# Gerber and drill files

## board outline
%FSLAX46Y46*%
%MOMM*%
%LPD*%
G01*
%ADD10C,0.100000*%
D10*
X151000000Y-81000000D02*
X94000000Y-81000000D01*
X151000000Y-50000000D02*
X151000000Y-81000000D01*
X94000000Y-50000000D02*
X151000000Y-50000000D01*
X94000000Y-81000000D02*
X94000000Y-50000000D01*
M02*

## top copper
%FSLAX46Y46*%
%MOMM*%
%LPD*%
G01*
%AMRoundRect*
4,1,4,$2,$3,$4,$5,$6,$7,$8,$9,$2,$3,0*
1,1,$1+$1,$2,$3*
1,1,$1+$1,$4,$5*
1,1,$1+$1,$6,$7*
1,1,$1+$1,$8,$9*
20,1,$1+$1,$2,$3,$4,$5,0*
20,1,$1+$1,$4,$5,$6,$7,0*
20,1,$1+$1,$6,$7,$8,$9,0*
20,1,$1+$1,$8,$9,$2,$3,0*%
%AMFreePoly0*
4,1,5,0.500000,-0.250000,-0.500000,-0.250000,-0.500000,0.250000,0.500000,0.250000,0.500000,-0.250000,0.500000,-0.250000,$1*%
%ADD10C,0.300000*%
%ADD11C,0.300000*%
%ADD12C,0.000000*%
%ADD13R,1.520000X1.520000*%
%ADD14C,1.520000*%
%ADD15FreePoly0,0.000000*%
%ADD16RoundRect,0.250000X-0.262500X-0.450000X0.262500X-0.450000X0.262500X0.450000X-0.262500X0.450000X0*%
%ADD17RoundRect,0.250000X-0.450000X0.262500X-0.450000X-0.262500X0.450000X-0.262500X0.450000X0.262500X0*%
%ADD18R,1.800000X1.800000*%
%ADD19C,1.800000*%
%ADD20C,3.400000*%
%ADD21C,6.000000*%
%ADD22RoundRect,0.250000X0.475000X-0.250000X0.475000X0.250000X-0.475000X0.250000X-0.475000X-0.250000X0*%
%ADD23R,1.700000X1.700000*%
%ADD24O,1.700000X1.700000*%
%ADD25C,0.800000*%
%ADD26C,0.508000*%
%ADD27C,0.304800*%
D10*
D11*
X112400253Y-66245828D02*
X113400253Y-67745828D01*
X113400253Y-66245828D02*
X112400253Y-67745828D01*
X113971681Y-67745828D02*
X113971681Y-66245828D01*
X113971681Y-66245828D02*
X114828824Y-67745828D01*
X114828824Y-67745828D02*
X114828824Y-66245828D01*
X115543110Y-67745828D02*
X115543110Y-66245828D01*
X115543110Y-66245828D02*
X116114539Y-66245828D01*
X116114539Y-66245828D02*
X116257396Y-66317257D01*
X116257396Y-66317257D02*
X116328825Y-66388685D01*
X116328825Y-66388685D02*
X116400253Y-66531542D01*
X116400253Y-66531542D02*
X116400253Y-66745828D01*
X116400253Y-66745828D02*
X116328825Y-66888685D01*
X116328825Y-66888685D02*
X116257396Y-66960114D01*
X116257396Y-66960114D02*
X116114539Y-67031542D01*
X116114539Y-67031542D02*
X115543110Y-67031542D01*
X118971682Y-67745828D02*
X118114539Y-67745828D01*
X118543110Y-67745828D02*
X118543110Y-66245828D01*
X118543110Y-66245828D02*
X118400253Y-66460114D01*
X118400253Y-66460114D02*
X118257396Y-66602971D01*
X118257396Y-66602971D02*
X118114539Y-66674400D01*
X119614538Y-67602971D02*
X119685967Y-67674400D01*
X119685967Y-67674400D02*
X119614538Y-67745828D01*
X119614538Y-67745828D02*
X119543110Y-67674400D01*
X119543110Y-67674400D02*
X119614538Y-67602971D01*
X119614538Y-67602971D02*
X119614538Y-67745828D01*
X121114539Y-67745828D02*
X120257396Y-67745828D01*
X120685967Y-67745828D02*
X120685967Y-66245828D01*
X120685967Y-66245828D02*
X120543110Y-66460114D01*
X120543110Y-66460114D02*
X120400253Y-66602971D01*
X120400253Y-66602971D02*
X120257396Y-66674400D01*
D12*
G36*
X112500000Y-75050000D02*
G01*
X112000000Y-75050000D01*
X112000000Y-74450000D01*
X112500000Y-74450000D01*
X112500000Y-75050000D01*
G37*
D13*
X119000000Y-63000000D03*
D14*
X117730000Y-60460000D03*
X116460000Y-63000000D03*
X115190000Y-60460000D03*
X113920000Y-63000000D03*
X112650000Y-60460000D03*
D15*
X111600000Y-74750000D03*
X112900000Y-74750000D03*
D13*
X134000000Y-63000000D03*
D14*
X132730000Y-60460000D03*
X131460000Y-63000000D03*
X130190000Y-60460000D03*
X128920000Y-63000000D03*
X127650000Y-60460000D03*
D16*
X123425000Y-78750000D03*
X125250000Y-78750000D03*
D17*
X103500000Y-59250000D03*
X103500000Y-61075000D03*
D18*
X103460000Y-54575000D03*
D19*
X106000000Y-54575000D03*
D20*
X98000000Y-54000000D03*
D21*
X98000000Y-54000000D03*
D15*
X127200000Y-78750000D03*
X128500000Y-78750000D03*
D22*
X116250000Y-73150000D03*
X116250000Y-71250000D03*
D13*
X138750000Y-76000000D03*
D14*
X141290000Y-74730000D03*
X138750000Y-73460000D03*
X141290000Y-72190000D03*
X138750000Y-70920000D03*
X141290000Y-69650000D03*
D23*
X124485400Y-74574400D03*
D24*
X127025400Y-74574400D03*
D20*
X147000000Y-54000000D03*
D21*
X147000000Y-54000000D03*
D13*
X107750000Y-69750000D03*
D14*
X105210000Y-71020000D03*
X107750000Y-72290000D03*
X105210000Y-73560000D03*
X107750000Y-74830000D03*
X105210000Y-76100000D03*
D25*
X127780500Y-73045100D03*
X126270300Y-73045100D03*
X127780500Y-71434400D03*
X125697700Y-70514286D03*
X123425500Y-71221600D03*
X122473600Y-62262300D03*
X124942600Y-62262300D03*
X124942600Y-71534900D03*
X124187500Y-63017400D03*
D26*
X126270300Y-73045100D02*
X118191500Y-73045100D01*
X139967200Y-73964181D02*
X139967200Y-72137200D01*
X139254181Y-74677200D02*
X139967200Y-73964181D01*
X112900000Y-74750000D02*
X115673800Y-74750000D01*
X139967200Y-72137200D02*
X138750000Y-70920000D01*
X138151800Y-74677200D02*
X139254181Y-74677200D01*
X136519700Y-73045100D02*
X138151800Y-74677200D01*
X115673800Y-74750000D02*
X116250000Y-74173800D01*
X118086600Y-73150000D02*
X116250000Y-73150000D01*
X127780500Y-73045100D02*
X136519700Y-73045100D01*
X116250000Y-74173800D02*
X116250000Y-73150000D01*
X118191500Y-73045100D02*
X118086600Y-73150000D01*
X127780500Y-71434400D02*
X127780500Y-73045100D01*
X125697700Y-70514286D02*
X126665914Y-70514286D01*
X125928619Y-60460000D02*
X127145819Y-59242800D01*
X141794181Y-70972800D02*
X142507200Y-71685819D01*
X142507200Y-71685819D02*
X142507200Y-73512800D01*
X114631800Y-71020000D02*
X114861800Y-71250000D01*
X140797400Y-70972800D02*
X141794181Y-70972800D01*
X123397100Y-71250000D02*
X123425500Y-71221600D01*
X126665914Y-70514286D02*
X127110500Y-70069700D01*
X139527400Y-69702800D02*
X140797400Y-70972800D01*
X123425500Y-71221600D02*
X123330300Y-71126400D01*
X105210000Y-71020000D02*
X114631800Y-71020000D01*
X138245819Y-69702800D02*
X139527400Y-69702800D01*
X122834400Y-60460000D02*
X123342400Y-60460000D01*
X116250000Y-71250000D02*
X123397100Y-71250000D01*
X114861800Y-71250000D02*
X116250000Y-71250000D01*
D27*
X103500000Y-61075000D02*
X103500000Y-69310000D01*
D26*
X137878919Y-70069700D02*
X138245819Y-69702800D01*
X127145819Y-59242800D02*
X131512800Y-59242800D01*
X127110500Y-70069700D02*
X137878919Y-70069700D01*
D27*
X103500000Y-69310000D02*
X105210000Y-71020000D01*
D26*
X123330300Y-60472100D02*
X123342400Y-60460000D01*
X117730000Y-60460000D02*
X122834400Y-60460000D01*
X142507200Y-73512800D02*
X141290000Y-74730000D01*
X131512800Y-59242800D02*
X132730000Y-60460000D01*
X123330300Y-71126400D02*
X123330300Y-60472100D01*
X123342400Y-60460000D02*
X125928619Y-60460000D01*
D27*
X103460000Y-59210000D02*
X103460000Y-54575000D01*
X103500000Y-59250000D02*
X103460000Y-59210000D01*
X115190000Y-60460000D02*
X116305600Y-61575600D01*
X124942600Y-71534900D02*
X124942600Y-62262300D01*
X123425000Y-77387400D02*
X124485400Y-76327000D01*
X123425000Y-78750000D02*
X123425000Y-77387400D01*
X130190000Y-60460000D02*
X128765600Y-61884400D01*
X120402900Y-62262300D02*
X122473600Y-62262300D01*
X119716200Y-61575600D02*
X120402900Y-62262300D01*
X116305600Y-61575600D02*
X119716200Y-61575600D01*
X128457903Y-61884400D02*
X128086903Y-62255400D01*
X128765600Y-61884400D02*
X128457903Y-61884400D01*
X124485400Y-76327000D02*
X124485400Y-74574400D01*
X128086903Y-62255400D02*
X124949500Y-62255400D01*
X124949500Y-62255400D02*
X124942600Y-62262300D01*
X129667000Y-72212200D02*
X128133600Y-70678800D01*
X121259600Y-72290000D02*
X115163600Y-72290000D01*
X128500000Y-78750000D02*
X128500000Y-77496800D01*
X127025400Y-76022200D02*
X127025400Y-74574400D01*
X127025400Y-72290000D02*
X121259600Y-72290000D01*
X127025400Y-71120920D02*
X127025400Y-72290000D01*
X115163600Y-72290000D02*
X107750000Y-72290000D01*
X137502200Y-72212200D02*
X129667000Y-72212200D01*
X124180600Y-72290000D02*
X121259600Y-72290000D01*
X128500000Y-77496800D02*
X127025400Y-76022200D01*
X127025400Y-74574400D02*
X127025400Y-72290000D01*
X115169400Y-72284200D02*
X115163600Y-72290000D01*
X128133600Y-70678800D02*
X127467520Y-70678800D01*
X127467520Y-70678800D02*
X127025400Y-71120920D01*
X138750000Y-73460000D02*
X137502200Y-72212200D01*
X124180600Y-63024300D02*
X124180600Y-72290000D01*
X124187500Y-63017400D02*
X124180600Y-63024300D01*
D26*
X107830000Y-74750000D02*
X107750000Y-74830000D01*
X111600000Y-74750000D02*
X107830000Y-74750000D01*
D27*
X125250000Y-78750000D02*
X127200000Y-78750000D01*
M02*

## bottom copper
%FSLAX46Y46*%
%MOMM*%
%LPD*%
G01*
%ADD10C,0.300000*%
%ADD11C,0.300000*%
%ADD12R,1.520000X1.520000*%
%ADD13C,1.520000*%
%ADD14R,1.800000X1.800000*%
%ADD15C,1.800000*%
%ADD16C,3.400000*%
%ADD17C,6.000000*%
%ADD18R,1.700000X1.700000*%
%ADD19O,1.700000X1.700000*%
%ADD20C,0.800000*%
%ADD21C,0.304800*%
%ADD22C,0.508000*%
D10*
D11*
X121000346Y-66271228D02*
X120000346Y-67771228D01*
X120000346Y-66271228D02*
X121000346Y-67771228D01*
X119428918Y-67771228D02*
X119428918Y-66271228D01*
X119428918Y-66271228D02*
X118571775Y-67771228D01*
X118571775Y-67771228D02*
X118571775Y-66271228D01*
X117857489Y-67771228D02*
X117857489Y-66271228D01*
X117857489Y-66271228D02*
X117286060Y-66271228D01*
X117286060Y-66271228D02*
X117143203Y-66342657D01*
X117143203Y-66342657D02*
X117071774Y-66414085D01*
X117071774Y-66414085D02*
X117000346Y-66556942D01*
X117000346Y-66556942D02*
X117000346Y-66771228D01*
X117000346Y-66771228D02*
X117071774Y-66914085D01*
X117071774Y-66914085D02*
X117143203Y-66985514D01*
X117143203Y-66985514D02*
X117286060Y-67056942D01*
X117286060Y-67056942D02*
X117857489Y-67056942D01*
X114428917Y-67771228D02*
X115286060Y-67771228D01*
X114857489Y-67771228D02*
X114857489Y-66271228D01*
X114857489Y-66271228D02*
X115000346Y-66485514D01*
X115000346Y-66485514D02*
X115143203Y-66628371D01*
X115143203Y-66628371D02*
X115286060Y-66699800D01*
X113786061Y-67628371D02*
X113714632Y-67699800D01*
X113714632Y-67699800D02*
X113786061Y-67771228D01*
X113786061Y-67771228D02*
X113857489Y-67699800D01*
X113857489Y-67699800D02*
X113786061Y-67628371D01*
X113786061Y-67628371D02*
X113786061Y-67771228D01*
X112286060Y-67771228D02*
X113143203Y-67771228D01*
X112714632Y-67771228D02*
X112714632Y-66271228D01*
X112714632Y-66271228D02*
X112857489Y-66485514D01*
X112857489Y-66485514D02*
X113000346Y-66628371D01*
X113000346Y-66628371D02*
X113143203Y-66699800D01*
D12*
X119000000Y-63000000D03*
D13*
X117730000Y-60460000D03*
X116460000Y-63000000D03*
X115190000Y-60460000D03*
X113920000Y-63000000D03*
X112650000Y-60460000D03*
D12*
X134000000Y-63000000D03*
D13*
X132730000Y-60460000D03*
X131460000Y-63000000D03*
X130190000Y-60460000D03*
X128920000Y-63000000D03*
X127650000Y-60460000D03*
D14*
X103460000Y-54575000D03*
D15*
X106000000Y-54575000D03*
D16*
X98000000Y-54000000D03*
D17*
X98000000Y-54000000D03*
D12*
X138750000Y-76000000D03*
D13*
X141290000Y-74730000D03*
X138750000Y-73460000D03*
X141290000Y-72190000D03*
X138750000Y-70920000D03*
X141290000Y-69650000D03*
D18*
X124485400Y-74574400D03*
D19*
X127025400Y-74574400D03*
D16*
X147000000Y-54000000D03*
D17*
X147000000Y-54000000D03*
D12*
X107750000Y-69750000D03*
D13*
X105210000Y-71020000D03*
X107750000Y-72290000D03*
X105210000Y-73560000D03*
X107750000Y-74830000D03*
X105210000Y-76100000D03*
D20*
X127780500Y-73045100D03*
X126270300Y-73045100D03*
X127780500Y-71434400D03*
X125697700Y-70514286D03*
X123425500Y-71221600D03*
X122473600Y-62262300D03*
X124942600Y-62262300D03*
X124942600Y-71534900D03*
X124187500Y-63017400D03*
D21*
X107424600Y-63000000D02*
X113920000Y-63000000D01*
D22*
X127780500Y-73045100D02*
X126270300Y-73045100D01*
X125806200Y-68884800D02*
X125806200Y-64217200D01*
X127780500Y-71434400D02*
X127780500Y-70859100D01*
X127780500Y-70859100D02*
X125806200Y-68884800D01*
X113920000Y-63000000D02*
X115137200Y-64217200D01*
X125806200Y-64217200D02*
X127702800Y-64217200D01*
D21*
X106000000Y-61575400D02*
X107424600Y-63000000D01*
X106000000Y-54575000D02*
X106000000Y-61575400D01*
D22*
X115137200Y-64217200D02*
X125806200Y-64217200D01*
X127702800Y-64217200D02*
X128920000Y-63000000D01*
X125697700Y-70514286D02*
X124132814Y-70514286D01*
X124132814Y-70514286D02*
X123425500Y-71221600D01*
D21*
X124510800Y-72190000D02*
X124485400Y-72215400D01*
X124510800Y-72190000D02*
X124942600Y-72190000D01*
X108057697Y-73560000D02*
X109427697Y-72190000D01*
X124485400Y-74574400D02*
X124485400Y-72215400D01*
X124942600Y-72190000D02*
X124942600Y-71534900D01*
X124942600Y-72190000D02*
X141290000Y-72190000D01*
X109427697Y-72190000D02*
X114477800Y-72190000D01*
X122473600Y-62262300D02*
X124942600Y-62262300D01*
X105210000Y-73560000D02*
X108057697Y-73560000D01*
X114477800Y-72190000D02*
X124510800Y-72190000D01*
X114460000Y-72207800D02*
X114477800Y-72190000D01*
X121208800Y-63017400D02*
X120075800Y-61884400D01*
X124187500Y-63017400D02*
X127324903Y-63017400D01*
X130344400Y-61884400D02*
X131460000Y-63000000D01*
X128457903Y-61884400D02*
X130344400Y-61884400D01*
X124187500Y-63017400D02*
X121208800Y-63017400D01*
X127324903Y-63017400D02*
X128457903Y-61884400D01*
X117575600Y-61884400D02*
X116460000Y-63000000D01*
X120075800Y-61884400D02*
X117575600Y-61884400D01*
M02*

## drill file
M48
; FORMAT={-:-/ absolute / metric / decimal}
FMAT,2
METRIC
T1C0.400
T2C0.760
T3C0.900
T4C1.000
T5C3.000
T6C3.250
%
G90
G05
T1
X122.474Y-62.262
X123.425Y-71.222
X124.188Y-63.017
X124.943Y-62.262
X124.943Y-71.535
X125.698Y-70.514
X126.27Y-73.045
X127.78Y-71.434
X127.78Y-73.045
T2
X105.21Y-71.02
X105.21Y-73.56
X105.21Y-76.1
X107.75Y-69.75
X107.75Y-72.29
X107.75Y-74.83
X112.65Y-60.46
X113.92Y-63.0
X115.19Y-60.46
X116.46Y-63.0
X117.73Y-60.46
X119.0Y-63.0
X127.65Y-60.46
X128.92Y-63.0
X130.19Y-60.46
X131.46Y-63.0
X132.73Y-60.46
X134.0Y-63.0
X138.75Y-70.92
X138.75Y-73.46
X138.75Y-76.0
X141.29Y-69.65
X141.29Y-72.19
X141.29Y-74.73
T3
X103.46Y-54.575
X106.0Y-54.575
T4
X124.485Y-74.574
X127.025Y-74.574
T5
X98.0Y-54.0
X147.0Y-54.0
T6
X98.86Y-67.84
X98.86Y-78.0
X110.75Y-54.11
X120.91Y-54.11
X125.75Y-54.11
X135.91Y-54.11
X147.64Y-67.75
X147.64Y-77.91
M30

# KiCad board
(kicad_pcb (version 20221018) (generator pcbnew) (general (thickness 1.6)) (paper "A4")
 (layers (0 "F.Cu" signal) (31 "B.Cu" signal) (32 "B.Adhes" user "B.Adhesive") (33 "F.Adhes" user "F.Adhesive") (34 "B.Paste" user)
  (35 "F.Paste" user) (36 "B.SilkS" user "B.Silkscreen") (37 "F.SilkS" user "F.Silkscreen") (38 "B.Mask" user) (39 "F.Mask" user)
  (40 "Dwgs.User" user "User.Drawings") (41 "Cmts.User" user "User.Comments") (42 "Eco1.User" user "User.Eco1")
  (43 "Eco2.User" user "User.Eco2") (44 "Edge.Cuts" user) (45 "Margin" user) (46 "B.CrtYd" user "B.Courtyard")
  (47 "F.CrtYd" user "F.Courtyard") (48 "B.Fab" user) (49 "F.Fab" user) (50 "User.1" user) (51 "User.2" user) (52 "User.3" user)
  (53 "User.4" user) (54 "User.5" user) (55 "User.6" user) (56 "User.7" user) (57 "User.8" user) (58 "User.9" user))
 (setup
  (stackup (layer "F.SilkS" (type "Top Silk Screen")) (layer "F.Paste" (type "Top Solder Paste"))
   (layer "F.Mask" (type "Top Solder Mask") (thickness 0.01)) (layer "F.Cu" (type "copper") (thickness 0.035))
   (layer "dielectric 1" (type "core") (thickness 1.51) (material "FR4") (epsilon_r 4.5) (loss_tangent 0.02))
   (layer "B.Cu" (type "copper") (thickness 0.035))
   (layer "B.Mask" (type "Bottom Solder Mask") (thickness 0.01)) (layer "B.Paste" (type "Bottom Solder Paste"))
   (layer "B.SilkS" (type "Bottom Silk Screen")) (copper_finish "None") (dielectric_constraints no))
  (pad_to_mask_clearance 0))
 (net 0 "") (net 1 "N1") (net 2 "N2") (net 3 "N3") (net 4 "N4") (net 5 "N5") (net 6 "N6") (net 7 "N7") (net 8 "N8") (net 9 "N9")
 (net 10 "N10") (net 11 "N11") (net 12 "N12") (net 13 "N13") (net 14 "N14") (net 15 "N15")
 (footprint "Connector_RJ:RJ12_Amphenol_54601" (layer "F.Cu") (at 119 63 180)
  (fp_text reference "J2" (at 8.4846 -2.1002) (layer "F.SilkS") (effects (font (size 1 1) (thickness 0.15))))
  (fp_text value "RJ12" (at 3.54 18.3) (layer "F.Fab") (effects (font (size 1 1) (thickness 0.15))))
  (pad "" np_thru_hole circle (at -1.91 8.89 180) (size 3.25 3.25) (drill 3.25) (layers "*.Cu" "*.Mask"))
  (pad "" np_thru_hole circle (at 8.25 8.89 180) (size 3.25 3.25) (drill 3.25) (layers "*.Cu" "*.Mask"))
  (pad "1" thru_hole rect (at 0 0 180) (size 1.52 1.52) (drill 0.76) (layers "*.Cu" "*.Mask") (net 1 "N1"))
  (pad "2" thru_hole circle (at 1.27 2.54 180) (size 1.52 1.52) (drill 0.76) (layers "*.Cu" "*.Mask") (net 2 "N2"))
  (pad "3" thru_hole circle (at 2.54 0 180) (size 1.52 1.52) (drill 0.76) (layers "*.Cu" "*.Mask") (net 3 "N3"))
  (pad "4" thru_hole circle (at 3.81 2.54 180) (size 1.52 1.52) (drill 0.76) (layers "*.Cu" "*.Mask") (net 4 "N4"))
  (pad "5" thru_hole circle (at 5.08 0 180) (size 1.52 1.52) (drill 0.76) (layers "*.Cu" "*.Mask") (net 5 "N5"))
  (pad "6" thru_hole circle (at 6.35 2.54 180) (size 1.52 1.52) (drill 0.76) (layers "*.Cu" "*.Mask") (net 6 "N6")))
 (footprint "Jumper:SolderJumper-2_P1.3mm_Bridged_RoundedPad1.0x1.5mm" (layer "F.Cu") (at 112.25 74.75) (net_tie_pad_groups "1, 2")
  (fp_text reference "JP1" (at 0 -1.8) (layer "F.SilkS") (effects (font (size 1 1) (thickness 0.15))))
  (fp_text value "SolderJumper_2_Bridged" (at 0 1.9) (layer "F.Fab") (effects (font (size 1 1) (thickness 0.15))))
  (fp_poly (pts (xy 0.25 -0.3) (xy -0.25 -0.3) (xy -0.25 0.3) (xy 0.25 0.3)) (stroke (width 0) (type solid)) (fill solid) (layer "F.Cu"))
  (pad "1" smd custom (at -0.65 0) (size 1 0.5) (layers "F.Cu" "F.Mask") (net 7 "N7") (zone_connect 2) (thermal_bridge_angle 45)
   (options (clearance outline) (anchor rect)) (primitives))
  (pad "2" smd custom (at 0.65 0) (size 1 0.5) (layers "F.Cu" "F.Mask") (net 5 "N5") (zone_connect 2) (thermal_bridge_angle 45)
   (options (clearance outline) (anchor rect)) (primitives)))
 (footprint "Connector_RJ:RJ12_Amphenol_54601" (layer "F.Cu") (at 134 63 180)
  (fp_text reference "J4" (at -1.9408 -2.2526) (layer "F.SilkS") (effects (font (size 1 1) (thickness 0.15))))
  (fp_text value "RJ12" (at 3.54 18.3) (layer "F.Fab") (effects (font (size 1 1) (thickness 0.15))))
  (pad "" np_thru_hole circle (at -1.91 8.89 180) (size 3.25 3.25) (drill 3.25) (layers "*.Cu" "*.Mask"))
  (pad "" np_thru_hole circle (at 8.25 8.89 180) (size 3.25 3.25) (drill 3.25) (layers "*.Cu" "*.Mask"))
  (pad "1" thru_hole rect (at 0 0 180) (size 1.52 1.52) (drill 0.76) (layers "*.Cu" "*.Mask") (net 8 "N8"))
  (pad "2" thru_hole circle (at 1.27 2.54 180) (size 1.52 1.52) (drill 0.76) (layers "*.Cu" "*.Mask") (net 2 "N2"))
  (pad "3" thru_hole circle (at 2.54 0 180) (size 1.52 1.52) (drill 0.76) (layers "*.Cu" "*.Mask") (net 3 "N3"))
  (pad "4" thru_hole circle (at 3.81 2.54 180) (size 1.52 1.52) (drill 0.76) (layers "*.Cu" "*.Mask") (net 4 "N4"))
  (pad "5" thru_hole circle (at 5.08 0 180) (size 1.52 1.52) (drill 0.76) (layers "*.Cu" "*.Mask") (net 5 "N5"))
  (pad "6" thru_hole circle (at 6.35 2.54 180) (size 1.52 1.52) (drill 0.76) (layers "*.Cu" "*.Mask") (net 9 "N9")))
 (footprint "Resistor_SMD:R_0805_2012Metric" (layer "F.Cu") (at 124.3375 78.75)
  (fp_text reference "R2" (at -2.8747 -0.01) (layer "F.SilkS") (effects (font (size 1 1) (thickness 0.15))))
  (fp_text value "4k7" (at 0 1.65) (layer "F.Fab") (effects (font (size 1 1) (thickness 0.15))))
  (pad "1" smd roundrect (at -0.9125 0) (size 1.025 1.4) (layers "F.Cu" "F.Paste" "F.Mask") (roundrect_rratio 0.243902439) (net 4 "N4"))
  (pad "2" smd roundrect (at 0.9125 0) (size 1.025 1.4) (layers "F.Cu" "F.Paste" "F.Mask") (roundrect_rratio 0.243902439) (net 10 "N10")))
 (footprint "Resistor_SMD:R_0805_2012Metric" (layer "F.Cu") (at 103.5 60.1625 -90)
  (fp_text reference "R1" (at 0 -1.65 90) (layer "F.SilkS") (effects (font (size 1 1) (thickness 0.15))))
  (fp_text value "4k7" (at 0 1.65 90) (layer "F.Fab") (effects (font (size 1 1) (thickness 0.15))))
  (pad "1" smd roundrect (at -0.9125 0 270) (size 1.025 1.4) (layers "F.Cu" "F.Paste" "F.Mask") (roundrect_rratio 0.243902439)
   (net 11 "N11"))
  (pad "2" smd roundrect (at 0.9125 0 270) (size 1.025 1.4) (layers "F.Cu" "F.Paste" "F.Mask") (roundrect_rratio 0.243902439) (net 2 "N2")))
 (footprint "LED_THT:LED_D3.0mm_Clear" (layer "F.Cu") (at 103.46 54.575)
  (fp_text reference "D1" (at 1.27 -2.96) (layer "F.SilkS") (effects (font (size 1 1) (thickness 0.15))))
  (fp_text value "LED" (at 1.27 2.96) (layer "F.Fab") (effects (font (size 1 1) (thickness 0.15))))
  (pad "1" thru_hole rect (at 0 0) (size 1.8 1.8) (drill 0.9) (layers "*.Cu" "*.Mask") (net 11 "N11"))
  (pad "2" thru_hole circle (at 2.54 0) (size 1.8 1.8) (drill 0.9) (layers "*.Cu" "*.Mask") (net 5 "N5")))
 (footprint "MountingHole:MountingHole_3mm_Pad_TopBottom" (layer "F.Cu") (at 98 54)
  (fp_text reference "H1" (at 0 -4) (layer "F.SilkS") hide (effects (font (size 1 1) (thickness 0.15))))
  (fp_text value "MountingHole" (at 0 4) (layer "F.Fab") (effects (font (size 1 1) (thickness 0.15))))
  (pad "1" thru_hole circle (at 0 0) (size 3.4 3.4) (drill 3) (layers "*.Cu" "*.Mask"))
  (pad "1" connect circle (at 0 0) (size 6 6) (layers "F.Cu" "F.Mask"))
  (pad "1" connect circle (at 0 0) (size 6 6) (layers "B.Cu" "B.Mask")))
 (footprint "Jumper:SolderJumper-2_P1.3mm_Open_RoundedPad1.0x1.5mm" (layer "F.Cu") (at 127.85 78.75)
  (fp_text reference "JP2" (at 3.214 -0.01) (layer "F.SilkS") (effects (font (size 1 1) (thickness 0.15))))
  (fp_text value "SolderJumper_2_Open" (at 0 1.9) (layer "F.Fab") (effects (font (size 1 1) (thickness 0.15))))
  (pad "1" smd custom (at -0.65 0) (size 1 0.5) (layers "F.Cu" "F.Mask") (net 10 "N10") (zone_connect 2) (thermal_bridge_angle 45)
   (options (clearance outline) (anchor rect)) (primitives))
  (pad "2" smd custom (at 0.65 0) (size 1 0.5) (layers "F.Cu" "F.Mask") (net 3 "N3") (zone_connect 2) (thermal_bridge_angle 45)
   (options (clearance outline) (anchor rect)) (primitives)))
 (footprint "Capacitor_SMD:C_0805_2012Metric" (layer "F.Cu") (at 116.25 72.2 90)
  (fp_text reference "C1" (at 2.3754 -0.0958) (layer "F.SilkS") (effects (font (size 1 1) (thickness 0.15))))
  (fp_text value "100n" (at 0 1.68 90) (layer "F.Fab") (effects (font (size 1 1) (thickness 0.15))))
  (pad "1" smd roundrect (at -0.95 0 90) (size 1 1.45) (layers "F.Cu" "F.Paste" "F.Mask") (roundrect_rratio 0.25) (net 5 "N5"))
  (pad "2" smd roundrect (at 0.95 0 90) (size 1 1.45) (layers "F.Cu" "F.Paste" "F.Mask") (roundrect_rratio 0.25) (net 2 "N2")))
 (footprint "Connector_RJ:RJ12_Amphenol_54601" (layer "F.Cu") (at 138.75 76 90)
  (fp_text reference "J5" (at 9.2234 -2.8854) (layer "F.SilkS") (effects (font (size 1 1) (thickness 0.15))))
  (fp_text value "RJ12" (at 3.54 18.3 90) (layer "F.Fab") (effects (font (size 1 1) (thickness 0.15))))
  (pad "" np_thru_hole circle (at -1.91 8.89 90) (size 3.25 3.25) (drill 3.25) (layers "*.Cu" "*.Mask"))
  (pad "" np_thru_hole circle (at 8.25 8.89 90) (size 3.25 3.25) (drill 3.25) (layers "*.Cu" "*.Mask"))
  (pad "1" thru_hole rect (at 0 0 90) (size 1.52 1.52) (drill 0.76) (layers "*.Cu" "*.Mask") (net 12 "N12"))
  (pad "2" thru_hole circle (at 1.27 2.54 90) (size 1.52 1.52) (drill 0.76) (layers "*.Cu" "*.Mask") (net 2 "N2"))
  (pad "3" thru_hole circle (at 2.54 0 90) (size 1.52 1.52) (drill 0.76) (layers "*.Cu" "*.Mask") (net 3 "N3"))
  (pad "4" thru_hole circle (at 3.81 2.54 90) (size 1.52 1.52) (drill 0.76) (layers "*.Cu" "*.Mask") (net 4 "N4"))
  (pad "5" thru_hole circle (at 5.08 0 90) (size 1.52 1.52) (drill 0.76) (layers "*.Cu" "*.Mask") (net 5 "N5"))
  (pad "6" thru_hole circle (at 6.35 2.54 90) (size 1.52 1.52) (drill 0.76) (layers "*.Cu" "*.Mask") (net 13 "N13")))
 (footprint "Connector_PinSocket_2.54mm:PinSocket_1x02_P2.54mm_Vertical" (layer "F.Cu") (at 124.4854 74.5744 90)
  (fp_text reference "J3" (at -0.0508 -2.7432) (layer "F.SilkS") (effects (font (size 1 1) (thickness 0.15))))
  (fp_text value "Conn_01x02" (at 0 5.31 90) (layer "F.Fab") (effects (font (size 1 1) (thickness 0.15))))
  (pad "1" thru_hole rect (at 0 0 90) (size 1.7 1.7) (drill 1) (layers "*.Cu" "*.Mask") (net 4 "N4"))
  (pad "2" thru_hole oval (at 0 2.54 90) (size 1.7 1.7) (drill 1) (layers "*.Cu" "*.Mask") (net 3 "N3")))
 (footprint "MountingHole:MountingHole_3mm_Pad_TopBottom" (layer "F.Cu") (at 147 54)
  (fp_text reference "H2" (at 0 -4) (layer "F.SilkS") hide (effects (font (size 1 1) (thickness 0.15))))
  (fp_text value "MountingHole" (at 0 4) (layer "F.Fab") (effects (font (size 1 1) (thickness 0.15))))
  (pad "1" thru_hole circle (at 0 0) (size 3.4 3.4) (drill 3) (layers "*.Cu" "*.Mask"))
  (pad "1" connect circle (at 0 0) (size 6 6) (layers "F.Cu" "F.Mask"))
  (pad "1" connect circle (at 0 0) (size 6 6) (layers "B.Cu" "B.Mask")))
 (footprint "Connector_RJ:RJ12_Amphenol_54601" (layer "F.Cu") (at 107.75 69.75 -90)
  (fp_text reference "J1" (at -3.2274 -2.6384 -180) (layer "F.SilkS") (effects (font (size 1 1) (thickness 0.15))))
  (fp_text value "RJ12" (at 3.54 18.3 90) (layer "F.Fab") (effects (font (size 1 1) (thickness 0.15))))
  (pad "" np_thru_hole circle (at -1.91 8.89 270) (size 3.25 3.25) (drill 3.25) (layers "*.Cu" "*.Mask"))
  (pad "" np_thru_hole circle (at 8.25 8.89 270) (size 3.25 3.25) (drill 3.25) (layers "*.Cu" "*.Mask"))
  (pad "1" thru_hole rect (at 0 0 270) (size 1.52 1.52) (drill 0.76) (layers "*.Cu" "*.Mask") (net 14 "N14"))
  (pad "2" thru_hole circle (at 1.27 2.54 270) (size 1.52 1.52) (drill 0.76) (layers "*.Cu" "*.Mask") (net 2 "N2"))
  (pad "3" thru_hole circle (at 2.54 0 270) (size 1.52 1.52) (drill 0.76) (layers "*.Cu" "*.Mask") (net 3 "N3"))
  (pad "4" thru_hole circle (at 3.81 2.54 270) (size 1.52 1.52) (drill 0.76) (layers "*.Cu" "*.Mask") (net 4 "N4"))
  (pad "5" thru_hole circle (at 5.08 0 270) (size 1.52 1.52) (drill 0.76) (layers "*.Cu" "*.Mask") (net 7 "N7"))
  (pad "6" thru_hole circle (at 6.35 2.54 270) (size 1.52 1.52) (drill 0.76) (layers "*.Cu" "*.Mask") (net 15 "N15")))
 (gr_line (start 151 81) (end 94 81) (stroke (width 0.1) (type default)) (layer "Edge.Cuts"))
 (gr_line (start 151 50) (end 151 81) (stroke (width 0.1) (type default)) (layer "Edge.Cuts"))
 (gr_line (start 94 50) (end 151 50) (stroke (width 0.1) (type default)) (layer "Edge.Cuts"))
 (gr_line (start 94 81) (end 94 50) (stroke (width 0.1) (type default)) (layer "Edge.Cuts"))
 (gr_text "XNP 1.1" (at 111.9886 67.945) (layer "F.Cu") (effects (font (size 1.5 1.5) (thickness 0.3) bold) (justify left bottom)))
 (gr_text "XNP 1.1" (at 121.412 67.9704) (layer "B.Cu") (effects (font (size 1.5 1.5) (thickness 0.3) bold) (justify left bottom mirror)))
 (segment (start 126.2703 73.0451) (end 118.1915 73.0451) (width 0.508) (layer "F.Cu") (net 5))
 (segment (start 139.9672 73.964181) (end 139.9672 72.1372) (width 0.508) (layer "F.Cu") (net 5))
 (segment (start 139.254181 74.6772) (end 139.9672 73.964181) (width 0.508) (layer "F.Cu") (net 5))
 (segment (start 112.9 74.75) (end 115.6738 74.75) (width 0.508) (layer "F.Cu") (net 5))
 (segment (start 139.9672 72.1372) (end 138.75 70.92) (width 0.508) (layer "F.Cu") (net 5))
 (segment (start 138.1518 74.6772) (end 139.254181 74.6772) (width 0.508) (layer "F.Cu") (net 5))
 (segment (start 136.5197 73.0451) (end 138.1518 74.6772) (width 0.508) (layer "F.Cu") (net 5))
 (segment (start 115.6738 74.75) (end 116.25 74.1738) (width 0.508) (layer "F.Cu") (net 5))
 (segment (start 118.0866 73.15) (end 116.25 73.15) (width 0.508) (layer "F.Cu") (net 5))
 (segment (start 127.7805 73.0451) (end 136.5197 73.0451) (width 0.508) (layer "F.Cu") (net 5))
 (segment (start 116.25 74.1738) (end 116.25 73.15) (width 0.508) (layer "F.Cu") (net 5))
 (segment (start 118.1915 73.0451) (end 118.0866 73.15) (width 0.508) (layer "F.Cu") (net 5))
 (segment (start 127.7805 71.4344) (end 127.7805 73.0451) (width 0.508) (layer "F.Cu") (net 5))
 (via (at 127.7805 73.0451) (size 0.8) (drill 0.4) (layers "F.Cu" "B.Cu") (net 5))
 (via (at 126.2703 73.0451) (size 0.8) (drill 0.4) (layers "F.Cu" "B.Cu") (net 5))
 (via (at 127.7805 71.4344) (size 0.8) (drill 0.4) (layers "F.Cu" "B.Cu") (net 5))
 (segment (start 107.4246 63) (end 113.92 63) (width 0.3048) (layer "B.Cu") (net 5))
 (segment (start 127.7805 73.0451) (end 126.2703 73.0451) (width 0.508) (layer "B.Cu") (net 5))
 (segment (start 125.8062 68.8848) (end 125.8062 64.2172) (width 0.508) (layer "B.Cu") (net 5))
 (segment (start 127.7805 71.4344) (end 127.7805 70.8591) (width 0.508) (layer "B.Cu") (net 5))
 (segment (start 127.7805 70.8591) (end 125.8062 68.8848) (width 0.508) (layer "B.Cu") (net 5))
 (segment (start 113.92 63) (end 115.1372 64.2172) (width 0.508) (layer "B.Cu") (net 5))
 (segment (start 125.8062 64.2172) (end 127.7028 64.2172) (width 0.508) (layer "B.Cu") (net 5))
 (segment (start 106 61.5754) (end 107.4246 63) (width 0.3048) (layer "B.Cu") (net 5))
 (segment (start 106 54.575) (end 106 61.5754) (width 0.3048) (layer "B.Cu") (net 5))
 (segment (start 115.1372 64.2172) (end 125.8062 64.2172) (width 0.508) (layer "B.Cu") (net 5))
 (segment (start 127.7028 64.2172) (end 128.92 63) (width 0.508) (layer "B.Cu") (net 5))
 (segment (start 125.6977 70.514286) (end 126.665914 70.514286) (width 0.508) (layer "F.Cu") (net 2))
 (segment (start 125.928619 60.46) (end 127.145819 59.2428) (width 0.508) (layer "F.Cu") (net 2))
 (segment (start 141.794181 70.9728) (end 142.5072 71.685819) (width 0.508) (layer "F.Cu") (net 2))
 (segment (start 142.5072 71.685819) (end 142.5072 73.5128) (width 0.508) (layer "F.Cu") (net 2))
 (segment (start 114.6318 71.02) (end 114.8618 71.25) (width 0.508) (layer "F.Cu") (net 2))
 (segment (start 140.7974 70.9728) (end 141.794181 70.9728) (width 0.508) (layer "F.Cu") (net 2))
 (segment (start 123.3971 71.25) (end 123.4255 71.2216) (width 0.508) (layer "F.Cu") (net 2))
 (segment (start 126.665914 70.514286) (end 127.1105 70.0697) (width 0.508) (layer "F.Cu") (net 2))
 (segment (start 139.5274 69.7028) (end 140.7974 70.9728) (width 0.508) (layer "F.Cu") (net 2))
 (segment (start 123.4255 71.2216) (end 123.3303 71.1264) (width 0.508) (layer "F.Cu") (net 2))
 (segment (start 105.21 71.02) (end 114.6318 71.02) (width 0.508) (layer "F.Cu") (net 2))
 (segment (start 138.245819 69.7028) (end 139.5274 69.7028) (width 0.508) (layer "F.Cu") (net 2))
 (segment (start 122.8344 60.46) (end 123.3424 60.46) (width 0.508) (layer "F.Cu") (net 2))
 (segment (start 116.25 71.25) (end 123.3971 71.25) (width 0.508) (layer "F.Cu") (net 2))
 (segment (start 114.8618 71.25) (end 116.25 71.25) (width 0.508) (layer "F.Cu") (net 2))
 (segment (start 103.5 61.075) (end 103.5 69.31) (width 0.3048) (layer "F.Cu") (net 2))
 (segment (start 137.878919 70.0697) (end 138.245819 69.7028) (width 0.508) (layer "F.Cu") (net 2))
 (segment (start 127.145819 59.2428) (end 131.5128 59.2428) (width 0.508) (layer "F.Cu") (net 2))
 (segment (start 127.1105 70.0697) (end 137.878919 70.0697) (width 0.508) (layer "F.Cu") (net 2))
 (segment (start 103.5 69.31) (end 105.21 71.02) (width 0.3048) (layer "F.Cu") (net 2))
 (segment (start 123.3303 60.4721) (end 123.3424 60.46) (width 0.508) (layer "F.Cu") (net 2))
 (segment (start 117.73 60.46) (end 122.8344 60.46) (width 0.508) (layer "F.Cu") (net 2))
 (segment (start 142.5072 73.5128) (end 141.29 74.73) (width 0.508) (layer "F.Cu") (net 2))
 (segment (start 131.5128 59.2428) (end 132.73 60.46) (width 0.508) (layer "F.Cu") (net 2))
 (segment (start 123.3303 71.1264) (end 123.3303 60.4721) (width 0.508) (layer "F.Cu") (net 2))
 (segment (start 123.3424 60.46) (end 125.928619 60.46) (width 0.508) (layer "F.Cu") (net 2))
 (via (at 125.6977 70.514286) (size 0.8) (drill 0.4) (layers "F.Cu" "B.Cu") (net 2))
 (via (at 123.4255 71.2216) (size 0.8) (drill 0.4) (layers "F.Cu" "B.Cu") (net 2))
 (segment (start 125.6977 70.514286) (end 124.132814 70.514286) (width 0.508) (layer "B.Cu") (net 2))
 (segment (start 124.132814 70.514286) (end 123.4255 71.2216) (width 0.508) (layer "B.Cu") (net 2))
 (segment (start 103.46 59.21) (end 103.46 54.575) (width 0.3048) (layer "F.Cu") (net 11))
 (segment (start 103.5 59.25) (end 103.46 59.21) (width 0.3048) (layer "F.Cu") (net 11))
 (segment (start 115.19 60.46) (end 116.3056 61.5756) (width 0.3048) (layer "F.Cu") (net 4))
 (segment (start 124.9426 71.5349) (end 124.9426 62.2623) (width 0.3048) (layer "F.Cu") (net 4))
 (segment (start 123.425 77.3874) (end 124.4854 76.327) (width 0.3048) (layer "F.Cu") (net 4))
 (segment (start 123.425 78.75) (end 123.425 77.3874) (width 0.3048) (layer "F.Cu") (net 4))
 (segment (start 130.19 60.46) (end 128.7656 61.8844) (width 0.3048) (layer "F.Cu") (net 4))
 (segment (start 120.4029 62.2623) (end 122.4736 62.2623) (width 0.3048) (layer "F.Cu") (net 4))
 (segment (start 119.7162 61.5756) (end 120.4029 62.2623) (width 0.3048) (layer "F.Cu") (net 4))
 (segment (start 116.3056 61.5756) (end 119.7162 61.5756) (width 0.3048) (layer "F.Cu") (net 4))
 (segment (start 128.457903 61.8844) (end 128.086903 62.2554) (width 0.3048) (layer "F.Cu") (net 4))
 (segment (start 128.7656 61.8844) (end 128.457903 61.8844) (width 0.3048) (layer "F.Cu") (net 4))
 (segment (start 124.4854 76.327) (end 124.4854 74.5744) (width 0.3048) (layer "F.Cu") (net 4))
 (segment (start 128.086903 62.2554) (end 124.9495 62.2554) (width 0.3048) (layer "F.Cu") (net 4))
 (segment (start 124.9495 62.2554) (end 124.9426 62.2623) (width 0.3048) (layer "F.Cu") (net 4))
 (via (at 122.4736 62.2623) (size 0.8) (drill 0.4) (layers "F.Cu" "B.Cu") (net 4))
 (via (at 124.9426 62.2623) (size 0.8) (drill 0.4) (layers "F.Cu" "B.Cu") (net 4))
 (via (at 124.9426 71.5349) (size 0.8) (drill 0.4) (layers "F.Cu" "B.Cu") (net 4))
 (segment (start 124.5108 72.19) (end 124.4854 72.2154) (width 0.3048) (layer "B.Cu") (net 4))
 (segment (start 124.5108 72.19) (end 124.9426 72.19) (width 0.3048) (layer "B.Cu") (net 4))
 (segment (start 108.057697 73.56) (end 109.427697 72.19) (width 0.3048) (layer "B.Cu") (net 4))
 (segment (start 124.4854 74.5744) (end 124.4854 72.2154) (width 0.3048) (layer "B.Cu") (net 4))
 (segment (start 124.9426 72.19) (end 124.9426 71.5349) (width 0.3048) (layer "B.Cu") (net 4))
 (segment (start 124.9426 72.19) (end 141.29 72.19) (width 0.3048) (layer "B.Cu") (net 4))
 (segment (start 109.427697 72.19) (end 114.4778 72.19) (width 0.3048) (layer "B.Cu") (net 4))
 (segment (start 122.4736 62.2623) (end 124.9426 62.2623) (width 0.3048) (layer "B.Cu") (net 4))
 (segment (start 105.21 73.56) (end 108.057697 73.56) (width 0.3048) (layer "B.Cu") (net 4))
 (segment (start 114.4778 72.19) (end 124.5108 72.19) (width 0.3048) (layer "B.Cu") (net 4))
 (segment (start 114.46 72.2078) (end 114.4778 72.19) (width 0.3048) (layer "B.Cu") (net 4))
 (segment (start 129.667 72.2122) (end 128.1336 70.6788) (width 0.3048) (layer "F.Cu") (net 3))
 (segment (start 121.2596 72.29) (end 115.1636 72.29) (width 0.3048) (layer "F.Cu") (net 3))
 (segment (start 128.5 78.75) (end 128.5 77.4968) (width 0.3048) (layer "F.Cu") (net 3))
 (segment (start 127.0254 76.0222) (end 127.0254 74.5744) (width 0.3048) (layer "F.Cu") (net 3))
 (segment (start 127.0254 72.29) (end 121.2596 72.29) (width 0.3048) (layer "F.Cu") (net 3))
 (segment (start 127.0254 71.12092) (end 127.0254 72.29) (width 0.3048) (layer "F.Cu") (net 3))
 (segment (start 115.1636 72.29) (end 107.75 72.29) (width 0.3048) (layer "F.Cu") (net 3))
 (segment (start 137.5022 72.2122) (end 129.667 72.2122) (width 0.3048) (layer "F.Cu") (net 3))
 (segment (start 124.1806 72.29) (end 121.2596 72.29) (width 0.3048) (layer "F.Cu") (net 3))
 (segment (start 128.5 77.4968) (end 127.0254 76.0222) (width 0.3048) (layer "F.Cu") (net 3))
 (segment (start 127.0254 74.5744) (end 127.0254 72.29) (width 0.3048) (layer "F.Cu") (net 3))
 (segment (start 115.1694 72.2842) (end 115.1636 72.29) (width 0.3048) (layer "F.Cu") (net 3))
 (segment (start 128.1336 70.6788) (end 127.46752 70.6788) (width 0.3048) (layer "F.Cu") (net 3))
 (segment (start 127.46752 70.6788) (end 127.0254 71.12092) (width 0.3048) (layer "F.Cu") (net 3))
 (segment (start 138.75 73.46) (end 137.5022 72.2122) (width 0.3048) (layer "F.Cu") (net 3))
 (segment (start 124.1806 63.0243) (end 124.1806 72.29) (width 0.3048) (layer "F.Cu") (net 3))
 (segment (start 124.1875 63.0174) (end 124.1806 63.0243) (width 0.3048) (layer "F.Cu") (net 3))
 (via (at 124.1875 63.0174) (size 0.8) (drill 0.4) (layers "F.Cu" "B.Cu") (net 3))
 (segment (start 121.2088 63.0174) (end 120.0758 61.8844) (width 0.3048) (layer "B.Cu") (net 3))
 (segment (start 124.1875 63.0174) (end 127.324903 63.0174) (width 0.3048) (layer "B.Cu") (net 3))
 (segment (start 130.3444 61.8844) (end 131.46 63) (width 0.3048) (layer "B.Cu") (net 3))
 (segment (start 128.457903 61.8844) (end 130.3444 61.8844) (width 0.3048) (layer "B.Cu") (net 3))
 (segment (start 124.1875 63.0174) (end 121.2088 63.0174) (width 0.3048) (layer "B.Cu") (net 3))
 (segment (start 127.324903 63.0174) (end 128.457903 61.8844) (width 0.3048) (layer "B.Cu") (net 3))
 (segment (start 117.5756 61.8844) (end 116.46 63) (width 0.3048) (layer "B.Cu") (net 3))
 (segment (start 120.0758 61.8844) (end 117.5756 61.8844) (width 0.3048) (layer "B.Cu") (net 3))
 (segment (start 107.83 74.75) (end 107.75 74.83) (width 0.508) (layer "F.Cu") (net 7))
 (segment (start 111.6 74.75) (end 107.83 74.75) (width 0.508) (layer "F.Cu") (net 7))
 (segment (start 125.25 78.75) (end 127.2 78.75) (width 0.3048) (layer "F.Cu") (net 10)))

